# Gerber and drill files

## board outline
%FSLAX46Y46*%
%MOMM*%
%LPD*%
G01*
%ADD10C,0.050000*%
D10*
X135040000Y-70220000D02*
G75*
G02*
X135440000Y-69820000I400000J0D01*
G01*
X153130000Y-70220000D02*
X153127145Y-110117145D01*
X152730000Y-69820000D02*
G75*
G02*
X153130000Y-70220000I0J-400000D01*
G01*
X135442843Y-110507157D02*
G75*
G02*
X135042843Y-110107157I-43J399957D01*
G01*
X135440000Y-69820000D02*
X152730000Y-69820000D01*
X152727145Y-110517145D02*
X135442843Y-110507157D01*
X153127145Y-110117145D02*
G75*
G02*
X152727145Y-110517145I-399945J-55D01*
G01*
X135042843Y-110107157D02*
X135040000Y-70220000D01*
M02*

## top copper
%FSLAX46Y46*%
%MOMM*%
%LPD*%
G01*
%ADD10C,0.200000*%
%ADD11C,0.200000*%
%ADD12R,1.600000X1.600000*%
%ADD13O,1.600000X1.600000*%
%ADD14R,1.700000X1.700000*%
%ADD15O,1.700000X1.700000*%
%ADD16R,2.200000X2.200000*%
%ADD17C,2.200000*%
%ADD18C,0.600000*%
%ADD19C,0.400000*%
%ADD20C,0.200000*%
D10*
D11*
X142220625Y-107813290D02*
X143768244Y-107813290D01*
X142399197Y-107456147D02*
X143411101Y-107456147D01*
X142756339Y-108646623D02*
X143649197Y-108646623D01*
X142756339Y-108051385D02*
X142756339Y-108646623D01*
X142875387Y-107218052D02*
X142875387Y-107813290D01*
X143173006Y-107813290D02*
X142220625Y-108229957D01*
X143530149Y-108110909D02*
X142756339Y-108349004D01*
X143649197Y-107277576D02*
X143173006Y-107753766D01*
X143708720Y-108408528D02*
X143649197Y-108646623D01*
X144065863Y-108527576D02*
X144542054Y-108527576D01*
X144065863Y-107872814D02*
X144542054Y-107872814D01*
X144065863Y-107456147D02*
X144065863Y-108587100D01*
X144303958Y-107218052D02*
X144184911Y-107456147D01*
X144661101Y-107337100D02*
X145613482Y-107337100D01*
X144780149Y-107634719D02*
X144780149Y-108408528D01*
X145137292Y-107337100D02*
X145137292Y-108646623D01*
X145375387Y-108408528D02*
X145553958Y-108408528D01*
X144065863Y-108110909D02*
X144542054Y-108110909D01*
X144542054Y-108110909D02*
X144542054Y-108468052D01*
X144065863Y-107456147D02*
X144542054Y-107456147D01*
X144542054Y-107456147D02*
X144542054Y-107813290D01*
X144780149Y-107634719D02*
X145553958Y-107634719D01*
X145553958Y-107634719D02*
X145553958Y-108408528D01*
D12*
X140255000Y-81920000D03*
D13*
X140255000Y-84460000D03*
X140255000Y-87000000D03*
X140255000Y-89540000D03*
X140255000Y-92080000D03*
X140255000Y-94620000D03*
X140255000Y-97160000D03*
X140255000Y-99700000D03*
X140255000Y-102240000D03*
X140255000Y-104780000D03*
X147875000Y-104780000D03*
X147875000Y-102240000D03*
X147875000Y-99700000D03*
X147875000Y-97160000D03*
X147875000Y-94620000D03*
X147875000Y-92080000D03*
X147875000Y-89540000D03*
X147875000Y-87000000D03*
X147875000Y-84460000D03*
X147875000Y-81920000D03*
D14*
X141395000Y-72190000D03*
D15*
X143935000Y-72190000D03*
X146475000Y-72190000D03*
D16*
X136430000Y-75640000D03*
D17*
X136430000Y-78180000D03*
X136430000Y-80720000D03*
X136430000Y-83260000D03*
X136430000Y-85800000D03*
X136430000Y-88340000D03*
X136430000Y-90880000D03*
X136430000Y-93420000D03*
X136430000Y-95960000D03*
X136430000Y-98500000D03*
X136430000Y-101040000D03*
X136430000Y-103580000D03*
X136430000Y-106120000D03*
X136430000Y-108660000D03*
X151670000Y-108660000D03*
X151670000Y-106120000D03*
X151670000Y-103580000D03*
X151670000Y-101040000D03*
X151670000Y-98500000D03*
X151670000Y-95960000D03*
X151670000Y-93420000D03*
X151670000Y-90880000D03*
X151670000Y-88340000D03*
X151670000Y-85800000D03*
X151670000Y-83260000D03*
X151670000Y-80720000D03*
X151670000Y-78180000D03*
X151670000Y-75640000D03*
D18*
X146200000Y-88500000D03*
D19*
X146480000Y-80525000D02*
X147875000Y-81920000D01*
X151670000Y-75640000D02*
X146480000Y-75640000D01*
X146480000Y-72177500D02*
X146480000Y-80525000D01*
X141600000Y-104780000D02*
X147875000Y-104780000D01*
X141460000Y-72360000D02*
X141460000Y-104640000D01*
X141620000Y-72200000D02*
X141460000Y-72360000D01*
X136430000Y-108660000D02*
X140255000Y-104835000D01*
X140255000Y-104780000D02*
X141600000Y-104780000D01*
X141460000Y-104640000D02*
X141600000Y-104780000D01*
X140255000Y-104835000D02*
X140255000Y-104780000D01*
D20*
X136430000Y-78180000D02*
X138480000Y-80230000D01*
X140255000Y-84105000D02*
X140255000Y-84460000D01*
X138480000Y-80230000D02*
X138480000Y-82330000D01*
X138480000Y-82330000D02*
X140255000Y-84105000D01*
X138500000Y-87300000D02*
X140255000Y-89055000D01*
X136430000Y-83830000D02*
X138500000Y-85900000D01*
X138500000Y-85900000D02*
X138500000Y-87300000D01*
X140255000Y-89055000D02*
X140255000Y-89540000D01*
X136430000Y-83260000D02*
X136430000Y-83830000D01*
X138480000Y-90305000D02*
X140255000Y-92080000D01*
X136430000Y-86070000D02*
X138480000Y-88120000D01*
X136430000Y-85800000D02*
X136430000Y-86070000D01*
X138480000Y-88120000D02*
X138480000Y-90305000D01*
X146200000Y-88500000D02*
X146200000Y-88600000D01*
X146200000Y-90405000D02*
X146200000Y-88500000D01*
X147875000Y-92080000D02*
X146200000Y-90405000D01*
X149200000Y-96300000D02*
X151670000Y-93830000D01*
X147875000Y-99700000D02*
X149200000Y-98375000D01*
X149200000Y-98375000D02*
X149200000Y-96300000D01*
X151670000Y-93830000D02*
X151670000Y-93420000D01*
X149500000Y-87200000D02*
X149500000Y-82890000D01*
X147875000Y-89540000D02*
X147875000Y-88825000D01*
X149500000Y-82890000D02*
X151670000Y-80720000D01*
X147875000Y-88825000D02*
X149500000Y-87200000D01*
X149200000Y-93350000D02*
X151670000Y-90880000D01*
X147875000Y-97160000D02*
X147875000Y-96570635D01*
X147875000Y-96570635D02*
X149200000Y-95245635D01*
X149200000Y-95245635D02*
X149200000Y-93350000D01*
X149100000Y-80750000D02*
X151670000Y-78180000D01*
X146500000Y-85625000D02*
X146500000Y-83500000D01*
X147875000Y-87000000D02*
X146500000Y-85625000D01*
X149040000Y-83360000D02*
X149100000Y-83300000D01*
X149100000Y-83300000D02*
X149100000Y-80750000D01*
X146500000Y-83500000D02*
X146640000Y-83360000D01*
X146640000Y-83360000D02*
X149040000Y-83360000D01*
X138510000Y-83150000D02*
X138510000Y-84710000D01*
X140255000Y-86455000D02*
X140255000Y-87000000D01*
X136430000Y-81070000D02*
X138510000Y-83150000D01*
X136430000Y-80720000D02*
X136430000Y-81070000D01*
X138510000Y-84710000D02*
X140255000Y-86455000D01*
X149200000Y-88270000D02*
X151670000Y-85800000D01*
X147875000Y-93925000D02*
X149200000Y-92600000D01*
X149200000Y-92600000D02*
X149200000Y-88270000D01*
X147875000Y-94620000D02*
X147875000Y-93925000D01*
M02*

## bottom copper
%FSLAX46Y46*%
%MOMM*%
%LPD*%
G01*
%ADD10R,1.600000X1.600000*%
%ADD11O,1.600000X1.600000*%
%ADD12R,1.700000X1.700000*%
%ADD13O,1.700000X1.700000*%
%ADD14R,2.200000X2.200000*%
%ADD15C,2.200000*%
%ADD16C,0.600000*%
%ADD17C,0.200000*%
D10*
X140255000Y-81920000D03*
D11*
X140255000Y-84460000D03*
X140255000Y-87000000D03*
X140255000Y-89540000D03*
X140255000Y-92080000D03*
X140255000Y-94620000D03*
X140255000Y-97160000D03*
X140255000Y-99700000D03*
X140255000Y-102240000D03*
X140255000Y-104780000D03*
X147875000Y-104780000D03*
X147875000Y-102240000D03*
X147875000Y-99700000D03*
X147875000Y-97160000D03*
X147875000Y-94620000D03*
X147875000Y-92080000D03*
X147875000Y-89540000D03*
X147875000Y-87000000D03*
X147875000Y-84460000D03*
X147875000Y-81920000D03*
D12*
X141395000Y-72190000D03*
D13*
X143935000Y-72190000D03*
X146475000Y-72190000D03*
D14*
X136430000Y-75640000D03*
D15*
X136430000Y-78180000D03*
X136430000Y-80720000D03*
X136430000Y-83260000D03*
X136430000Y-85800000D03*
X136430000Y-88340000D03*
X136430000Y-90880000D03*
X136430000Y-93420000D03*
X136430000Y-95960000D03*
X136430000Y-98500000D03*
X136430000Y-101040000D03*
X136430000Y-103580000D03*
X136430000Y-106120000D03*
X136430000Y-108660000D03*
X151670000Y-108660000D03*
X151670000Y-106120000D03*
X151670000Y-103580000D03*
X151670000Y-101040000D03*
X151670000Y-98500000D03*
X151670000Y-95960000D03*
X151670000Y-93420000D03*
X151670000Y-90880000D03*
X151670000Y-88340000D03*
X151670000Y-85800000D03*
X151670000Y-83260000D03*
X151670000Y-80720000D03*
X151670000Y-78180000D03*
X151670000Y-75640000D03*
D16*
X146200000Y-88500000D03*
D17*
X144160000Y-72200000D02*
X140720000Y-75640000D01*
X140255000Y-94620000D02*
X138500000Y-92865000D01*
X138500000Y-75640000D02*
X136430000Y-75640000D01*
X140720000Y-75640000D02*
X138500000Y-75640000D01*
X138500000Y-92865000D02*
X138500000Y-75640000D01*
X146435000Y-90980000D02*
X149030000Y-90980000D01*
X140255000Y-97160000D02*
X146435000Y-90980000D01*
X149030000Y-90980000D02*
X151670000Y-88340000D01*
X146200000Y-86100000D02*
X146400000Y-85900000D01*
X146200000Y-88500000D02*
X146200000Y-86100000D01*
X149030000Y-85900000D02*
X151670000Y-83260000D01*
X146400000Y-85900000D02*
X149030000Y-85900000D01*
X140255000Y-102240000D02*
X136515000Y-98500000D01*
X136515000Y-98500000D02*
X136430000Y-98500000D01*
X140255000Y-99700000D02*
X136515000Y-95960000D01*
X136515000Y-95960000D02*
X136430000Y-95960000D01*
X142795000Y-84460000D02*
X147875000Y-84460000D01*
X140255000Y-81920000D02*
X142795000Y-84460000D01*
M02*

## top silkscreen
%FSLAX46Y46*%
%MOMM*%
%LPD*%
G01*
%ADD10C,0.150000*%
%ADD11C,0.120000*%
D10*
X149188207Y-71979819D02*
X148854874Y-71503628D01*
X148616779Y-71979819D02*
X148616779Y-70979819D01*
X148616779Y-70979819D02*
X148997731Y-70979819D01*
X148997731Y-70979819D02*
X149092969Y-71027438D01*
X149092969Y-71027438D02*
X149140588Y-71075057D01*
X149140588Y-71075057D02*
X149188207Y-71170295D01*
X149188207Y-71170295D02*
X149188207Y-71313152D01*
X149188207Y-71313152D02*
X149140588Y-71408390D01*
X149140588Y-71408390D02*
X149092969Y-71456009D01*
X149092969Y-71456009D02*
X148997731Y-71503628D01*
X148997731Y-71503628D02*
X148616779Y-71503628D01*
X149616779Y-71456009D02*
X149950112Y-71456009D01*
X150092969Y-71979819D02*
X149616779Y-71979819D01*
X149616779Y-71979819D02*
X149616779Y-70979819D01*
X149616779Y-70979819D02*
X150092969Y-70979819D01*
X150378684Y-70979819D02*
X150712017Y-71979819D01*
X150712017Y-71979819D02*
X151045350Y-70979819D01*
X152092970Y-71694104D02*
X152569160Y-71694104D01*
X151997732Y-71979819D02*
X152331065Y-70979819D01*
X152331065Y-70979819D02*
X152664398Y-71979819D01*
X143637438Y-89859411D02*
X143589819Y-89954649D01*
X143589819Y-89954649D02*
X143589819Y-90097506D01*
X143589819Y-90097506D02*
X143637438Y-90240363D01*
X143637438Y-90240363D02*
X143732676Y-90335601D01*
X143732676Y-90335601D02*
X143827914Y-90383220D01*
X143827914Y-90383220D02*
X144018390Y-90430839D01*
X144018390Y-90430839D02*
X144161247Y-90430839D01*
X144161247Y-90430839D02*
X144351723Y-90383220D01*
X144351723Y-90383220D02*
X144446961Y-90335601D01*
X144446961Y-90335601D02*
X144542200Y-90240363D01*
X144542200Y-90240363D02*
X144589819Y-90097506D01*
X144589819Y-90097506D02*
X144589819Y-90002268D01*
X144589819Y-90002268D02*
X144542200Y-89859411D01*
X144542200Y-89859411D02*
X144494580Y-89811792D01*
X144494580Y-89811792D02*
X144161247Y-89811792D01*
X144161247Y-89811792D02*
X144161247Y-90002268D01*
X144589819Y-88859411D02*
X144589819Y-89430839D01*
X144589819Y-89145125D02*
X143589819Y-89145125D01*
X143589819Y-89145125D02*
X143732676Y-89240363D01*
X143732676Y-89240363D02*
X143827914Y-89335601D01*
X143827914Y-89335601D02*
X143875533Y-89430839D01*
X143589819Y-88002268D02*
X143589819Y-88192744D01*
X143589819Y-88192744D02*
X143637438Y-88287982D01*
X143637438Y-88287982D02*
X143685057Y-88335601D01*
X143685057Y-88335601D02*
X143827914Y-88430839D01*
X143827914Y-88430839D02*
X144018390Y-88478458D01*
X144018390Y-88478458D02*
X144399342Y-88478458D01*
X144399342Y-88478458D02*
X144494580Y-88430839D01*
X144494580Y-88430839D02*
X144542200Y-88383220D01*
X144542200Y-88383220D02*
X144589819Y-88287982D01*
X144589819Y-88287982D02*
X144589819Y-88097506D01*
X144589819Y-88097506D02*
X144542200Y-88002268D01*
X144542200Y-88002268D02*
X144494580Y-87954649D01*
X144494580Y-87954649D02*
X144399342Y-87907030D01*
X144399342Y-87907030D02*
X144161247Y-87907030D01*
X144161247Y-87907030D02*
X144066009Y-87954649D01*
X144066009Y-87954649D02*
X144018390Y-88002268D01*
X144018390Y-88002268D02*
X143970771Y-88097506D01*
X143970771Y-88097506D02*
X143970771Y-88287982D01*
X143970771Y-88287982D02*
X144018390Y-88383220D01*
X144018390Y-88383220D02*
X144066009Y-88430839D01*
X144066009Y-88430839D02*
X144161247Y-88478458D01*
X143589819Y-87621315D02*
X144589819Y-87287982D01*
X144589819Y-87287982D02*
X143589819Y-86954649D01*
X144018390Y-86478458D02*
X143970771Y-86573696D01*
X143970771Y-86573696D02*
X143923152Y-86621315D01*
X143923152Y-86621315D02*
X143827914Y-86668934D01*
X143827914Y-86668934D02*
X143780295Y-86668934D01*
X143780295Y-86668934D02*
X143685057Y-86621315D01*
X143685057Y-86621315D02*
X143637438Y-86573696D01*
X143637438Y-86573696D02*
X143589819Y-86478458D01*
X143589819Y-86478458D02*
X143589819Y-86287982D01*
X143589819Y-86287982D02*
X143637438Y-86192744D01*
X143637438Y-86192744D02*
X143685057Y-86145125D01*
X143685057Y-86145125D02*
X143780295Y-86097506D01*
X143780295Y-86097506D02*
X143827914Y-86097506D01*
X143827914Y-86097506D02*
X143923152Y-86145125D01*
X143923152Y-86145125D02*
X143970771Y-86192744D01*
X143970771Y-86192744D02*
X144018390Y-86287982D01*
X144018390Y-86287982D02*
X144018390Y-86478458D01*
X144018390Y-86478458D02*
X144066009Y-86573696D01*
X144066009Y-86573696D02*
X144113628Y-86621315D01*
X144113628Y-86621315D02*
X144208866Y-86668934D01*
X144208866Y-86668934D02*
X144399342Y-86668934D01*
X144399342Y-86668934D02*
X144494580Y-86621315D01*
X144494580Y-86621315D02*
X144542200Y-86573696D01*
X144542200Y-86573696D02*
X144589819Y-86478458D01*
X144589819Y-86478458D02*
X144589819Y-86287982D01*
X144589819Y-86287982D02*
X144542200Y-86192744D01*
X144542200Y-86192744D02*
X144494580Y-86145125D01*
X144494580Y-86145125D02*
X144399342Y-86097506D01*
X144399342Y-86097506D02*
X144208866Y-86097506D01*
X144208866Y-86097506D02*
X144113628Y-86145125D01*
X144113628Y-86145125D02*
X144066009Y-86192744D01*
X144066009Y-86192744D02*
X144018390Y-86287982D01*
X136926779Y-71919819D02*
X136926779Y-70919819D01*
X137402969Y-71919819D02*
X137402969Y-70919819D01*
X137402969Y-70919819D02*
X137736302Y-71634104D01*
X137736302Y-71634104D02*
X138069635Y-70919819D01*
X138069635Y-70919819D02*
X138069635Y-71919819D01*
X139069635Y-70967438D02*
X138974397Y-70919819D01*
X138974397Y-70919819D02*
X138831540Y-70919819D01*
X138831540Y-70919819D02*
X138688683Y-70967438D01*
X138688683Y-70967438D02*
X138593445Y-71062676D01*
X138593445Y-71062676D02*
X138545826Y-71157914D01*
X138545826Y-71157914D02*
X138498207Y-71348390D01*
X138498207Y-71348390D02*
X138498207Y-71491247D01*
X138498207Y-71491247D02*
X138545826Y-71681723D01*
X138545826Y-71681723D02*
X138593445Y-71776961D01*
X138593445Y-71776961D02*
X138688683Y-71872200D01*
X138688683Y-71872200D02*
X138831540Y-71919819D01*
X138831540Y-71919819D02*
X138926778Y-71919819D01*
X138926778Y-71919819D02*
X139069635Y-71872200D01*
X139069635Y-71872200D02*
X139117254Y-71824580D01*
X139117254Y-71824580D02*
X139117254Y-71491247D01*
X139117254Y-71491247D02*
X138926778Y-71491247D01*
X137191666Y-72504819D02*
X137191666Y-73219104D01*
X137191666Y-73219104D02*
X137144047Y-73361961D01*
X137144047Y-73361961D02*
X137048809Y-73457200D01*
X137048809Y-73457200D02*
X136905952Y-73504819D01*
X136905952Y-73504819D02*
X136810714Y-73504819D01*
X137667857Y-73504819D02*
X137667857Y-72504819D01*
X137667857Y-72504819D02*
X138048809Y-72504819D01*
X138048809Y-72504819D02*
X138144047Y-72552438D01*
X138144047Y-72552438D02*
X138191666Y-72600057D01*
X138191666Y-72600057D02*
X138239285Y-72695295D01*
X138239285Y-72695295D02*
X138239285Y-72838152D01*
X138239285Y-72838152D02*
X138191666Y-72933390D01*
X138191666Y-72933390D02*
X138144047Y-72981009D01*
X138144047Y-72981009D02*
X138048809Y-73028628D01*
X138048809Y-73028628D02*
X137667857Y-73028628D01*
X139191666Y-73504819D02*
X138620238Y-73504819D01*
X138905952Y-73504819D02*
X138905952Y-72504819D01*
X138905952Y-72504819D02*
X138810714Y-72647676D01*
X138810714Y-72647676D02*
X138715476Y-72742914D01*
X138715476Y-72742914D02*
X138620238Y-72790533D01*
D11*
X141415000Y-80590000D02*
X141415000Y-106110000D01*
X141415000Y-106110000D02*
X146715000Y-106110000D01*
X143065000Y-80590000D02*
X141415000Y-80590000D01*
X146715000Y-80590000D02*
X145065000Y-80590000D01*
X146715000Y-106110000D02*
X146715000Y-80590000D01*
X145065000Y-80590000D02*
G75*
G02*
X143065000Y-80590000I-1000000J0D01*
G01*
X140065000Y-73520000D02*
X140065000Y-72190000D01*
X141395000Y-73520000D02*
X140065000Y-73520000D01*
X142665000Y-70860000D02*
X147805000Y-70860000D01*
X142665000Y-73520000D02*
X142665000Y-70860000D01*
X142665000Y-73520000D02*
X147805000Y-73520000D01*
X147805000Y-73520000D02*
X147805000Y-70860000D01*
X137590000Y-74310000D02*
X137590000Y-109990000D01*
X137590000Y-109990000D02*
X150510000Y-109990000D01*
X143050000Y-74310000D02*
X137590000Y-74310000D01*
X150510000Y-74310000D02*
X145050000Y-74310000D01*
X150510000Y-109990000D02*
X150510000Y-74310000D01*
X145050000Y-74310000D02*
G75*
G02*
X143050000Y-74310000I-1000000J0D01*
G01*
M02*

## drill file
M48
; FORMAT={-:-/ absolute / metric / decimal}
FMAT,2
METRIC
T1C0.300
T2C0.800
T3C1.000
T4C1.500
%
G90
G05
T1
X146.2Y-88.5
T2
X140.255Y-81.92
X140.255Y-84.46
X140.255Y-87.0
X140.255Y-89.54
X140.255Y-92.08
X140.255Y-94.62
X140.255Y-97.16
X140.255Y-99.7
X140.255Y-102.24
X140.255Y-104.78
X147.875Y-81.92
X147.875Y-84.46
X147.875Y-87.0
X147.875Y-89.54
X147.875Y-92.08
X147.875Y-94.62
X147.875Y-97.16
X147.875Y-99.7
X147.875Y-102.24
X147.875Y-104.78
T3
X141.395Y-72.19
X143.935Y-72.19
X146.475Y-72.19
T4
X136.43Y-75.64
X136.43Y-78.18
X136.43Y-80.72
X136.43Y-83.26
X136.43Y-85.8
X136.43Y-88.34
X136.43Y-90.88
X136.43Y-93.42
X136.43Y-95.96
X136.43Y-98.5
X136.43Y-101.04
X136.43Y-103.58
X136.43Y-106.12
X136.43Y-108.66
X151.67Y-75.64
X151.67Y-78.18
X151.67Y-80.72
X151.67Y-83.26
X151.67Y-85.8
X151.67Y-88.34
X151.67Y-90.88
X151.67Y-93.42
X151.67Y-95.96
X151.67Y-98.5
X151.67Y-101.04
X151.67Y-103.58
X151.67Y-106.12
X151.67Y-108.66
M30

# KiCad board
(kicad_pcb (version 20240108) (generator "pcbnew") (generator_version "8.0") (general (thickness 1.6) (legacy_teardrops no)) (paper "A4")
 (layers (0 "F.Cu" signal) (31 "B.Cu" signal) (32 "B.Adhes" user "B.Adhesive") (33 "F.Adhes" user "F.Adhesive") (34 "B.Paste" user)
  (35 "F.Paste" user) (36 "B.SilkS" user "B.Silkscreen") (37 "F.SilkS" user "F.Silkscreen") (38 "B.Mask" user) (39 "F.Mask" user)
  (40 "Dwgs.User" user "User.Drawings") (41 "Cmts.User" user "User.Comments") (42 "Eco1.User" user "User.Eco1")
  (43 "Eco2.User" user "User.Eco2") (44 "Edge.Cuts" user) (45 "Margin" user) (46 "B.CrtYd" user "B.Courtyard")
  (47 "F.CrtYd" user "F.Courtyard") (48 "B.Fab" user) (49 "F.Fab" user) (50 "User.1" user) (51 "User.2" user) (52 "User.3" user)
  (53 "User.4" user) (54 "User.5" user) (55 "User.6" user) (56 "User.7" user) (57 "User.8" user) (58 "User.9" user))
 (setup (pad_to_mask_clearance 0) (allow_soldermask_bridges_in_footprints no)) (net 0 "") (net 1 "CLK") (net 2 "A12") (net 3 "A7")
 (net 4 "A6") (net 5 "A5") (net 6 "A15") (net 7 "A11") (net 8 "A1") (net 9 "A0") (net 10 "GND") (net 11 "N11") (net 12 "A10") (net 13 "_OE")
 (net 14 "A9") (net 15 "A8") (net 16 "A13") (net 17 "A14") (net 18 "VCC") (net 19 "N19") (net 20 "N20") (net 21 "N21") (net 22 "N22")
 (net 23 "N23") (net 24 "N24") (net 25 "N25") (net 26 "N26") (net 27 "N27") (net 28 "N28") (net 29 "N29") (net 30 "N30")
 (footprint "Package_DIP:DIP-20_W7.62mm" (layer "F.Cu") (at 140.255 81.92)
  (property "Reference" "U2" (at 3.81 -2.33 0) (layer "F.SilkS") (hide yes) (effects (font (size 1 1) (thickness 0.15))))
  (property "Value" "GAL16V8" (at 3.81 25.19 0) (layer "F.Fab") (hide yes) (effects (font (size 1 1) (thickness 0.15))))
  (fp_line (start 1.16 -1.33) (end 1.16 24.19) (stroke (width 0.12) (type solid)) (layer "F.SilkS"))
  (fp_line (start 1.16 24.19) (end 6.46 24.19) (stroke (width 0.12) (type solid)) (layer "F.SilkS"))
  (fp_line (start 2.81 -1.33) (end 1.16 -1.33) (stroke (width 0.12) (type solid)) (layer "F.SilkS"))
  (fp_line (start 6.46 -1.33) (end 4.81 -1.33) (stroke (width 0.12) (type solid)) (layer "F.SilkS"))
  (fp_line (start 6.46 24.19) (end 6.46 -1.33) (stroke (width 0.12) (type solid)) (layer "F.SilkS"))
  (fp_arc (start 4.81 -1.33) (mid 3.81 -0.33) (end 2.81 -1.33) (stroke (width 0.12) (type solid)) (layer "F.SilkS"))
  (pad "1" thru_hole rect (at 0 0) (size 1.6 1.6) (drill 0.8) (layers "*.Cu" "*.Mask") (remove_unused_layers no) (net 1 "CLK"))
  (pad "2" thru_hole oval (at 0 2.54) (size 1.6 1.6) (drill 0.8) (layers "*.Cu" "*.Mask") (remove_unused_layers no) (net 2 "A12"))
  (pad "3" thru_hole oval (at 0 5.08) (size 1.6 1.6) (drill 0.8) (layers "*.Cu" "*.Mask") (remove_unused_layers no) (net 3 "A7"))
  (pad "4" thru_hole oval (at 0 7.62) (size 1.6 1.6) (drill 0.8) (layers "*.Cu" "*.Mask") (remove_unused_layers no) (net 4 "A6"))
  (pad "5" thru_hole oval (at 0 10.16) (size 1.6 1.6) (drill 0.8) (layers "*.Cu" "*.Mask") (remove_unused_layers no) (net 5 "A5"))
  (pad "6" thru_hole oval (at 0 12.7) (size 1.6 1.6) (drill 0.8) (layers "*.Cu" "*.Mask") (remove_unused_layers no) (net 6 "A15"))
  (pad "7" thru_hole oval (at 0 15.24) (size 1.6 1.6) (drill 0.8) (layers "*.Cu" "*.Mask") (remove_unused_layers no) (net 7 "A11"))
  (pad "8" thru_hole oval (at 0 17.78) (size 1.6 1.6) (drill 0.8) (layers "*.Cu" "*.Mask") (remove_unused_layers no) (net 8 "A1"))
  (pad "9" thru_hole oval (at 0 20.32) (size 1.6 1.6) (drill 0.8) (layers "*.Cu" "*.Mask") (remove_unused_layers no) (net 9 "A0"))
  (pad "10" thru_hole oval (at 0 22.86) (size 1.6 1.6) (drill 0.8) (layers "*.Cu" "*.Mask") (remove_unused_layers no) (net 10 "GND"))
  (pad "11" thru_hole oval (at 7.62 22.86) (size 1.6 1.6) (drill 0.8) (layers "*.Cu" "*.Mask") (remove_unused_layers no) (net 10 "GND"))
  (pad "12" thru_hole oval (at 7.62 20.32) (size 1.6 1.6) (drill 0.8) (layers "*.Cu" "*.Mask") (remove_unused_layers no) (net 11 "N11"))
  (pad "13" thru_hole oval (at 7.62 17.78) (size 1.6 1.6) (drill 0.8) (layers "*.Cu" "*.Mask") (remove_unused_layers no) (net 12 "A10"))
  (pad "14" thru_hole oval (at 7.62 15.24) (size 1.6 1.6) (drill 0.8) (layers "*.Cu" "*.Mask") (remove_unused_layers no) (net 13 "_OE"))
  (pad "15" thru_hole oval (at 7.62 12.7) (size 1.6 1.6) (drill 0.8) (layers "*.Cu" "*.Mask") (remove_unused_layers no) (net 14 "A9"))
  (pad "16" thru_hole oval (at 7.62 10.16) (size 1.6 1.6) (drill 0.8) (layers "*.Cu" "*.Mask") (remove_unused_layers no) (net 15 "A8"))
  (pad "17" thru_hole oval (at 7.62 7.62) (size 1.6 1.6) (drill 0.8) (layers "*.Cu" "*.Mask") (remove_unused_layers no) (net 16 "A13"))
  (pad "18" thru_hole oval (at 7.62 5.08) (size 1.6 1.6) (drill 0.8) (layers "*.Cu" "*.Mask") (remove_unused_layers no) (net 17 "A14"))
  (pad "19" thru_hole oval (at 7.62 2.54) (size 1.6 1.6) (drill 0.8) (layers "*.Cu" "*.Mask") (remove_unused_layers no) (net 1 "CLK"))
  (pad "20" thru_hole oval (at 7.62 0) (size 1.6 1.6) (drill 0.8) (layers "*.Cu" "*.Mask") (remove_unused_layers no) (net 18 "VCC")))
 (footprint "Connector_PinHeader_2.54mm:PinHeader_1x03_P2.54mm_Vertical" (layer "F.Cu") (at 141.395 72.19 90)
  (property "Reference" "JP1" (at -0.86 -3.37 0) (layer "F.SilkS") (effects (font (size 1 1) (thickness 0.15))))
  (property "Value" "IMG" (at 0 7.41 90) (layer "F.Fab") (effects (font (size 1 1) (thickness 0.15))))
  (fp_line (start -1.33 -1.33) (end 0 -1.33) (stroke (width 0.12) (type solid)) (layer "F.SilkS"))
  (fp_line (start -1.33 0) (end -1.33 -1.33) (stroke (width 0.12) (type solid)) (layer "F.SilkS"))
  (fp_line (start 1.33 1.27) (end 1.33 6.41) (stroke (width 0.12) (type solid)) (layer "F.SilkS"))
  (fp_line (start -1.33 1.27) (end 1.33 1.27) (stroke (width 0.12) (type solid)) (layer "F.SilkS"))
  (fp_line (start -1.33 1.27) (end -1.33 6.41) (stroke (width 0.12) (type solid)) (layer "F.SilkS"))
  (fp_line (start -1.33 6.41) (end 1.33 6.41) (stroke (width 0.12) (type solid)) (layer "F.SilkS"))
  (pad "1" thru_hole rect (at 0 0 90) (size 1.7 1.7) (drill 1) (layers "*.Cu" "*.Mask") (remove_unused_layers no) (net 10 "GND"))
  (pad "2" thru_hole oval (at 0 2.54 90) (size 1.7 1.7) (drill 1) (layers "*.Cu" "*.Mask") (remove_unused_layers no) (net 6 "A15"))
  (pad "3" thru_hole oval (at 0 5.08 90) (size 1.7 1.7) (drill 1) (layers "*.Cu" "*.Mask") (remove_unused_layers no) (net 18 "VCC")))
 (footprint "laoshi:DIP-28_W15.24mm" (layer "F.Cu") (at 136.43 75.64)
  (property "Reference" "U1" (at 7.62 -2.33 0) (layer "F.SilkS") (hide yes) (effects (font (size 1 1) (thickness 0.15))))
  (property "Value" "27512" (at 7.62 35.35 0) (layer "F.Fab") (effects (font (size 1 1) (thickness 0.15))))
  (fp_line (start 1.16 -1.33) (end 1.16 34.35) (stroke (width 0.12) (type solid)) (layer "F.SilkS"))
  (fp_line (start 1.16 34.35) (end 14.08 34.35) (stroke (width 0.12) (type solid)) (layer "F.SilkS"))
  (fp_line (start 6.62 -1.33) (end 1.16 -1.33) (stroke (width 0.12) (type solid)) (layer "F.SilkS"))
  (fp_line (start 14.08 -1.33) (end 8.62 -1.33) (stroke (width 0.12) (type solid)) (layer "F.SilkS"))
  (fp_line (start 14.08 34.35) (end 14.08 -1.33) (stroke (width 0.12) (type solid)) (layer "F.SilkS"))
  (fp_arc (start 8.62 -1.33) (mid 7.62 -0.33) (end 6.62 -1.33) (stroke (width 0.12) (type solid)) (layer "F.SilkS"))
  (pad "1" thru_hole rect (at 0 0) (size 2.2 2.2) (drill 1.5) (layers "*.Cu" "*.Mask") (remove_unused_layers no) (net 6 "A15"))
  (pad "2" thru_hole circle (at 0 2.54) (size 2.2 2.2) (drill 1.5) (layers "*.Cu" "*.Mask") (remove_unused_layers no) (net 2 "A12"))
  (pad "3" thru_hole circle (at 0 5.08) (size 2.2 2.2) (drill 1.5) (layers "*.Cu" "*.Mask") (remove_unused_layers no) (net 3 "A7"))
  (pad "4" thru_hole circle (at 0 7.62) (size 2.2 2.2) (drill 1.5) (layers "*.Cu" "*.Mask") (remove_unused_layers no) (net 4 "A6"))
  (pad "5" thru_hole circle (at 0 10.16) (size 2.2 2.2) (drill 1.5) (layers "*.Cu" "*.Mask") (remove_unused_layers no) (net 5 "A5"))
  (pad "6" thru_hole circle (at 0 12.7) (size 2.2 2.2) (drill 1.5) (layers "*.Cu" "*.Mask") (remove_unused_layers no) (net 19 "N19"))
  (pad "7" thru_hole circle (at 0 15.24) (size 2.2 2.2) (drill 1.5) (layers "*.Cu" "*.Mask") (remove_unused_layers no) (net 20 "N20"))
  (pad "8" thru_hole circle (at 0 17.78) (size 2.2 2.2) (drill 1.5) (layers "*.Cu" "*.Mask") (remove_unused_layers no) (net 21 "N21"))
  (pad "9" thru_hole circle (at 0 20.32) (size 2.2 2.2) (drill 1.5) (layers "*.Cu" "*.Mask") (remove_unused_layers no) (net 8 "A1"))
  (pad "10" thru_hole circle (at 0 22.86) (size 2.2 2.2) (drill 1.5) (layers "*.Cu" "*.Mask") (remove_unused_layers no) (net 9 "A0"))
  (pad "11" thru_hole circle (at 0 25.4) (size 2.2 2.2) (drill 1.5) (layers "*.Cu" "*.Mask") (remove_unused_layers no) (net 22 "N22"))
  (pad "12" thru_hole circle (at 0 27.94) (size 2.2 2.2) (drill 1.5) (layers "*.Cu" "*.Mask") (remove_unused_layers no) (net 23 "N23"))
  (pad "13" thru_hole circle (at 0 30.48) (size 2.2 2.2) (drill 1.5) (layers "*.Cu" "*.Mask") (remove_unused_layers no) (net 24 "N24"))
  (pad "14" thru_hole circle (at 0 33.02) (size 2.2 2.2) (drill 1.5) (layers "*.Cu" "*.Mask") (remove_unused_layers no) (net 10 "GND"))
  (pad "15" thru_hole circle (at 15.24 33.02) (size 2.2 2.2) (drill 1.5) (layers "*.Cu" "*.Mask") (remove_unused_layers no) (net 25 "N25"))
  (pad "16" thru_hole circle (at 15.24 30.48) (size 2.2 2.2) (drill 1.5) (layers "*.Cu" "*.Mask") (remove_unused_layers no) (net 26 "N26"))
  (pad "17" thru_hole circle (at 15.24 27.94) (size 2.2 2.2) (drill 1.5) (layers "*.Cu" "*.Mask") (remove_unused_layers no) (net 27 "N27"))
  (pad "18" thru_hole circle (at 15.24 25.4) (size 2.2 2.2) (drill 1.5) (layers "*.Cu" "*.Mask") (remove_unused_layers no) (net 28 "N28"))
  (pad "19" thru_hole circle (at 15.24 22.86) (size 2.2 2.2) (drill 1.5) (layers "*.Cu" "*.Mask") (remove_unused_layers no) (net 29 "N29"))
  (pad "20" thru_hole circle (at 15.24 20.32) (size 2.2 2.2) (drill 1.5) (layers "*.Cu" "*.Mask") (remove_unused_layers no) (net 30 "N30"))
  (pad "21" thru_hole circle (at 15.24 17.78) (size 2.2 2.2) (drill 1.5) (layers "*.Cu" "*.Mask") (remove_unused_layers no) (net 12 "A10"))
  (pad "22" thru_hole circle (at 15.24 15.24) (size 2.2 2.2) (drill 1.5) (layers "*.Cu" "*.Mask") (remove_unused_layers no) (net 13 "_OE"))
  (pad "23" thru_hole circle (at 15.24 12.7) (size 2.2 2.2) (drill 1.5) (layers "*.Cu" "*.Mask") (remove_unused_layers no) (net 7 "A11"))
  (pad "24" thru_hole circle (at 15.24 10.16) (size 2.2 2.2) (drill 1.5) (layers "*.Cu" "*.Mask") (remove_unused_layers no) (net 14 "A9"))
  (pad "25" thru_hole circle (at 15.24 7.62) (size 2.2 2.2) (drill 1.5) (layers "*.Cu" "*.Mask") (remove_unused_layers no) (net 15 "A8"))
  (pad "26" thru_hole circle (at 15.24 5.08) (size 2.2 2.2) (drill 1.5) (layers "*.Cu" "*.Mask") (remove_unused_layers no) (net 16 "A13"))
  (pad "27" thru_hole circle (at 15.24 2.54) (size 2.2 2.2) (drill 1.5) (layers "*.Cu" "*.Mask") (remove_unused_layers no) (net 17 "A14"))
  (pad "28" thru_hole circle (at 15.24 0) (size 2.2 2.2) (drill 1.5) (layers "*.Cu" "*.Mask") (remove_unused_layers no) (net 18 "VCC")))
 (gr_arc (start 135.04 70.22) (mid 135.157145 69.937145) (end 135.44 69.82) (stroke (width 0.05) (type default)) (layer "Edge.Cuts"))
 (gr_line (start 153.13 70.22) (end 153.127145 110.117145) (stroke (width 0.05) (type default)) (layer "Edge.Cuts"))
 (gr_arc (start 152.73 69.82) (mid 153.012855 69.937145) (end 153.13 70.22) (stroke (width 0.05) (type default)) (layer "Edge.Cuts"))
 (gr_arc (start 135.442843 110.507157) (mid 135.159988 110.390012) (end 135.042843 110.107157) (stroke (width 0.05) (type default))
  (layer "Edge.Cuts"))
 (gr_line (start 135.44 69.82) (end 152.73 69.82) (stroke (width 0.05) (type default)) (layer "Edge.Cuts"))
 (gr_line (start 152.727145 110.517145) (end 135.442843 110.507157) (stroke (width 0.05) (type default)) (layer "Edge.Cuts"))
 (gr_arc (start 153.127145 110.117145) (mid 153.01 110.4) (end 152.727145 110.517145) (stroke (width 0.05) (type default))
  (layer "Edge.Cuts"))
 (gr_line (start 135.042843 110.107157) (end 135.04 70.22) (stroke (width 0.05) (type default)) (layer "Edge.Cuts"))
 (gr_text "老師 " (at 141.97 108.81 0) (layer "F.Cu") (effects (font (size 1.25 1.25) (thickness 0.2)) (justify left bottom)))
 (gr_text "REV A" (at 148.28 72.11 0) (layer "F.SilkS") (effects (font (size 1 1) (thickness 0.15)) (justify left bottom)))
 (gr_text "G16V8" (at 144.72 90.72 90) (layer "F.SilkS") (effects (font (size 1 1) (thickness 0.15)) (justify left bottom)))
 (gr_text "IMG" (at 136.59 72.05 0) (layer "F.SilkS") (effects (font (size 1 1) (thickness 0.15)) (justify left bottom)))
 (segment (start 144.16 72.2) (end 140.72 75.64) (width 0.2) (layer "B.Cu") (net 6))
 (segment (start 140.255 94.62) (end 138.5 92.865) (width 0.2) (layer "B.Cu") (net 6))
 (segment (start 138.5 75.64) (end 136.43 75.64) (width 0.2) (layer "B.Cu") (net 6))
 (segment (start 140.72 75.64) (end 138.5 75.64) (width 0.2) (layer "B.Cu") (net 6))
 (segment (start 138.5 92.865) (end 138.5 75.64) (width 0.2) (layer "B.Cu") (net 6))
 (segment (start 146.48 80.525) (end 147.875 81.92) (width 0.4) (layer "F.Cu") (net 18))
 (segment (start 151.67 75.64) (end 146.48 75.64) (width 0.4) (layer "F.Cu") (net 18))
 (segment (start 146.48 72.1775) (end 146.48 80.525) (width 0.4) (layer "F.Cu") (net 18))
 (segment (start 141.6 104.78) (end 147.875 104.78) (width 0.4) (layer "F.Cu") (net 10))
 (segment (start 141.46 72.36) (end 141.46 104.64) (width 0.4) (layer "F.Cu") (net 10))
 (segment (start 141.62 72.2) (end 141.46 72.36) (width 0.4) (layer "F.Cu") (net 10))
 (segment (start 136.43 108.66) (end 140.255 104.835) (width 0.4) (layer "F.Cu") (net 10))
 (segment (start 140.255 104.78) (end 141.6 104.78) (width 0.4) (layer "F.Cu") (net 10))
 (segment (start 141.46 104.64) (end 141.6 104.78) (width 0.4) (layer "F.Cu") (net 10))
 (segment (start 140.255 104.835) (end 140.255 104.78) (width 0.4) (layer "F.Cu") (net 10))
 (segment (start 136.43 78.18) (end 138.48 80.23) (width 0.2) (layer "F.Cu") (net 2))
 (segment (start 140.255 84.105) (end 140.255 84.46) (width 0.2) (layer "F.Cu") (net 2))
 (segment (start 138.48 80.23) (end 138.48 82.33) (width 0.2) (layer "F.Cu") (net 2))
 (segment (start 138.48 82.33) (end 140.255 84.105) (width 0.2) (layer "F.Cu") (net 2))
 (segment (start 138.5 87.3) (end 140.255 89.055) (width 0.2) (layer "F.Cu") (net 4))
 (segment (start 136.43 83.83) (end 138.5 85.9) (width 0.2) (layer "F.Cu") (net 4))
 (segment (start 138.5 85.9) (end 138.5 87.3) (width 0.2) (layer "F.Cu") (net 4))
 (segment (start 140.255 89.055) (end 140.255 89.54) (width 0.2) (layer "F.Cu") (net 4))
 (segment (start 136.43 83.26) (end 136.43 83.83) (width 0.2) (layer "F.Cu") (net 4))
 (segment (start 138.48 90.305) (end 140.255 92.08) (width 0.2) (layer "F.Cu") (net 5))
 (segment (start 136.43 86.07) (end 138.48 88.12) (width 0.2) (layer "F.Cu") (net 5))
 (segment (start 136.43 85.8) (end 136.43 86.07) (width 0.2) (layer "F.Cu") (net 5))
 (segment (start 138.48 88.12) (end 138.48 90.305) (width 0.2) (layer "F.Cu") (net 5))
 (segment (start 146.435 90.98) (end 149.03 90.98) (width 0.2) (layer "B.Cu") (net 7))
 (segment (start 140.255 97.16) (end 146.435 90.98) (width 0.2) (layer "B.Cu") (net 7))
 (segment (start 149.03 90.98) (end 151.67 88.34) (width 0.2) (layer "B.Cu") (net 7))
 (segment (start 146.2 88.5) (end 146.2 88.6) (width 0.2) (layer "F.Cu") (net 15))
 (segment (start 146.2 90.405) (end 146.2 88.5) (width 0.2) (layer "F.Cu") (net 15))
 (segment (start 147.875 92.08) (end 146.2 90.405) (width 0.2) (layer "F.Cu") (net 15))
 (via (at 146.2 88.5) (size 0.6) (drill 0.3) (layers "F.Cu" "B.Cu") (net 15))
 (segment (start 146.2 86.1) (end 146.4 85.9) (width 0.2) (layer "B.Cu") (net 15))
 (segment (start 146.2 88.5) (end 146.2 86.1) (width 0.2) (layer "B.Cu") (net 15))
 (segment (start 149.03 85.9) (end 151.67 83.26) (width 0.2) (layer "B.Cu") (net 15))
 (segment (start 146.4 85.9) (end 149.03 85.9) (width 0.2) (layer "B.Cu") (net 15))
 (segment (start 140.255 102.24) (end 136.515 98.5) (width 0.2) (layer "B.Cu") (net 9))
 (segment (start 136.515 98.5) (end 136.43 98.5) (width 0.2) (layer "B.Cu") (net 9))
 (segment (start 149.2 96.3) (end 151.67 93.83) (width 0.2) (layer "F.Cu") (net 12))
 (segment (start 147.875 99.7) (end 149.2 98.375) (width 0.2) (layer "F.Cu") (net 12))
 (segment (start 149.2 98.375) (end 149.2 96.3) (width 0.2) (layer "F.Cu") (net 12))
 (segment (start 151.67 93.83) (end 151.67 93.42) (width 0.2) (layer "F.Cu") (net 12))
 (segment (start 140.255 99.7) (end 136.515 95.96) (width 0.2) (layer "B.Cu") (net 8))
 (segment (start 136.515 95.96) (end 136.43 95.96) (width 0.2) (layer "B.Cu") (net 8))
 (segment (start 149.5 87.2) (end 149.5 82.89) (width 0.2) (layer "F.Cu") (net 16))
 (segment (start 147.875 89.54) (end 147.875 88.825) (width 0.2) (layer "F.Cu") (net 16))
 (segment (start 149.5 82.89) (end 151.67 80.72) (width 0.2) (layer "F.Cu") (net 16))
 (segment (start 147.875 88.825) (end 149.5 87.2) (width 0.2) (layer "F.Cu") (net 16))
 (segment (start 149.2 93.35) (end 151.67 90.88) (width 0.2) (layer "F.Cu") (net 13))
 (segment (start 147.875 97.16) (end 147.875 96.570635) (width 0.2) (layer "F.Cu") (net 13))
 (segment (start 147.875 96.570635) (end 149.2 95.245635) (width 0.2) (layer "F.Cu") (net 13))
 (segment (start 149.2 95.245635) (end 149.2 93.35) (width 0.2) (layer "F.Cu") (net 13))
 (segment (start 149.1 80.75) (end 151.67 78.18) (width 0.2) (layer "F.Cu") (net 17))
 (segment (start 146.5 85.625) (end 146.5 83.5) (width 0.2) (layer "F.Cu") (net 17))
 (segment (start 147.875 87) (end 146.5 85.625) (width 0.2) (layer "F.Cu") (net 17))
 (segment (start 149.04 83.36) (end 149.1 83.3) (width 0.2) (layer "F.Cu") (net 17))
 (segment (start 149.1 83.3) (end 149.1 80.75) (width 0.2) (layer "F.Cu") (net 17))
 (segment (start 146.5 83.5) (end 146.64 83.36) (width 0.2) (layer "F.Cu") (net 17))
 (segment (start 146.64 83.36) (end 149.04 83.36) (width 0.2) (layer "F.Cu") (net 17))
 (segment (start 138.51 83.15) (end 138.51 84.71) (width 0.2) (layer "F.Cu") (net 3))
 (segment (start 140.255 86.455) (end 140.255 87) (width 0.2) (layer "F.Cu") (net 3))
 (segment (start 136.43 81.07) (end 138.51 83.15) (width 0.2) (layer "F.Cu") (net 3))
 (segment (start 136.43 80.72) (end 136.43 81.07) (width 0.2) (layer "F.Cu") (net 3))
 (segment (start 138.51 84.71) (end 140.255 86.455) (width 0.2) (layer "F.Cu") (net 3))
 (segment (start 149.2 88.27) (end 151.67 85.8) (width 0.2) (layer "F.Cu") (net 14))
 (segment (start 147.875 93.925) (end 149.2 92.6) (width 0.2) (layer "F.Cu") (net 14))
 (segment (start 149.2 92.6) (end 149.2 88.27) (width 0.2) (layer "F.Cu") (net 14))
 (segment (start 147.875 94.62) (end 147.875 93.925) (width 0.2) (layer "F.Cu") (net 14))
 (segment (start 142.795 84.46) (end 147.875 84.46) (width 0.2) (layer "B.Cu") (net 1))
 (segment (start 140.255 81.92) (end 142.795 84.46) (width 0.2) (layer "B.Cu") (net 1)))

